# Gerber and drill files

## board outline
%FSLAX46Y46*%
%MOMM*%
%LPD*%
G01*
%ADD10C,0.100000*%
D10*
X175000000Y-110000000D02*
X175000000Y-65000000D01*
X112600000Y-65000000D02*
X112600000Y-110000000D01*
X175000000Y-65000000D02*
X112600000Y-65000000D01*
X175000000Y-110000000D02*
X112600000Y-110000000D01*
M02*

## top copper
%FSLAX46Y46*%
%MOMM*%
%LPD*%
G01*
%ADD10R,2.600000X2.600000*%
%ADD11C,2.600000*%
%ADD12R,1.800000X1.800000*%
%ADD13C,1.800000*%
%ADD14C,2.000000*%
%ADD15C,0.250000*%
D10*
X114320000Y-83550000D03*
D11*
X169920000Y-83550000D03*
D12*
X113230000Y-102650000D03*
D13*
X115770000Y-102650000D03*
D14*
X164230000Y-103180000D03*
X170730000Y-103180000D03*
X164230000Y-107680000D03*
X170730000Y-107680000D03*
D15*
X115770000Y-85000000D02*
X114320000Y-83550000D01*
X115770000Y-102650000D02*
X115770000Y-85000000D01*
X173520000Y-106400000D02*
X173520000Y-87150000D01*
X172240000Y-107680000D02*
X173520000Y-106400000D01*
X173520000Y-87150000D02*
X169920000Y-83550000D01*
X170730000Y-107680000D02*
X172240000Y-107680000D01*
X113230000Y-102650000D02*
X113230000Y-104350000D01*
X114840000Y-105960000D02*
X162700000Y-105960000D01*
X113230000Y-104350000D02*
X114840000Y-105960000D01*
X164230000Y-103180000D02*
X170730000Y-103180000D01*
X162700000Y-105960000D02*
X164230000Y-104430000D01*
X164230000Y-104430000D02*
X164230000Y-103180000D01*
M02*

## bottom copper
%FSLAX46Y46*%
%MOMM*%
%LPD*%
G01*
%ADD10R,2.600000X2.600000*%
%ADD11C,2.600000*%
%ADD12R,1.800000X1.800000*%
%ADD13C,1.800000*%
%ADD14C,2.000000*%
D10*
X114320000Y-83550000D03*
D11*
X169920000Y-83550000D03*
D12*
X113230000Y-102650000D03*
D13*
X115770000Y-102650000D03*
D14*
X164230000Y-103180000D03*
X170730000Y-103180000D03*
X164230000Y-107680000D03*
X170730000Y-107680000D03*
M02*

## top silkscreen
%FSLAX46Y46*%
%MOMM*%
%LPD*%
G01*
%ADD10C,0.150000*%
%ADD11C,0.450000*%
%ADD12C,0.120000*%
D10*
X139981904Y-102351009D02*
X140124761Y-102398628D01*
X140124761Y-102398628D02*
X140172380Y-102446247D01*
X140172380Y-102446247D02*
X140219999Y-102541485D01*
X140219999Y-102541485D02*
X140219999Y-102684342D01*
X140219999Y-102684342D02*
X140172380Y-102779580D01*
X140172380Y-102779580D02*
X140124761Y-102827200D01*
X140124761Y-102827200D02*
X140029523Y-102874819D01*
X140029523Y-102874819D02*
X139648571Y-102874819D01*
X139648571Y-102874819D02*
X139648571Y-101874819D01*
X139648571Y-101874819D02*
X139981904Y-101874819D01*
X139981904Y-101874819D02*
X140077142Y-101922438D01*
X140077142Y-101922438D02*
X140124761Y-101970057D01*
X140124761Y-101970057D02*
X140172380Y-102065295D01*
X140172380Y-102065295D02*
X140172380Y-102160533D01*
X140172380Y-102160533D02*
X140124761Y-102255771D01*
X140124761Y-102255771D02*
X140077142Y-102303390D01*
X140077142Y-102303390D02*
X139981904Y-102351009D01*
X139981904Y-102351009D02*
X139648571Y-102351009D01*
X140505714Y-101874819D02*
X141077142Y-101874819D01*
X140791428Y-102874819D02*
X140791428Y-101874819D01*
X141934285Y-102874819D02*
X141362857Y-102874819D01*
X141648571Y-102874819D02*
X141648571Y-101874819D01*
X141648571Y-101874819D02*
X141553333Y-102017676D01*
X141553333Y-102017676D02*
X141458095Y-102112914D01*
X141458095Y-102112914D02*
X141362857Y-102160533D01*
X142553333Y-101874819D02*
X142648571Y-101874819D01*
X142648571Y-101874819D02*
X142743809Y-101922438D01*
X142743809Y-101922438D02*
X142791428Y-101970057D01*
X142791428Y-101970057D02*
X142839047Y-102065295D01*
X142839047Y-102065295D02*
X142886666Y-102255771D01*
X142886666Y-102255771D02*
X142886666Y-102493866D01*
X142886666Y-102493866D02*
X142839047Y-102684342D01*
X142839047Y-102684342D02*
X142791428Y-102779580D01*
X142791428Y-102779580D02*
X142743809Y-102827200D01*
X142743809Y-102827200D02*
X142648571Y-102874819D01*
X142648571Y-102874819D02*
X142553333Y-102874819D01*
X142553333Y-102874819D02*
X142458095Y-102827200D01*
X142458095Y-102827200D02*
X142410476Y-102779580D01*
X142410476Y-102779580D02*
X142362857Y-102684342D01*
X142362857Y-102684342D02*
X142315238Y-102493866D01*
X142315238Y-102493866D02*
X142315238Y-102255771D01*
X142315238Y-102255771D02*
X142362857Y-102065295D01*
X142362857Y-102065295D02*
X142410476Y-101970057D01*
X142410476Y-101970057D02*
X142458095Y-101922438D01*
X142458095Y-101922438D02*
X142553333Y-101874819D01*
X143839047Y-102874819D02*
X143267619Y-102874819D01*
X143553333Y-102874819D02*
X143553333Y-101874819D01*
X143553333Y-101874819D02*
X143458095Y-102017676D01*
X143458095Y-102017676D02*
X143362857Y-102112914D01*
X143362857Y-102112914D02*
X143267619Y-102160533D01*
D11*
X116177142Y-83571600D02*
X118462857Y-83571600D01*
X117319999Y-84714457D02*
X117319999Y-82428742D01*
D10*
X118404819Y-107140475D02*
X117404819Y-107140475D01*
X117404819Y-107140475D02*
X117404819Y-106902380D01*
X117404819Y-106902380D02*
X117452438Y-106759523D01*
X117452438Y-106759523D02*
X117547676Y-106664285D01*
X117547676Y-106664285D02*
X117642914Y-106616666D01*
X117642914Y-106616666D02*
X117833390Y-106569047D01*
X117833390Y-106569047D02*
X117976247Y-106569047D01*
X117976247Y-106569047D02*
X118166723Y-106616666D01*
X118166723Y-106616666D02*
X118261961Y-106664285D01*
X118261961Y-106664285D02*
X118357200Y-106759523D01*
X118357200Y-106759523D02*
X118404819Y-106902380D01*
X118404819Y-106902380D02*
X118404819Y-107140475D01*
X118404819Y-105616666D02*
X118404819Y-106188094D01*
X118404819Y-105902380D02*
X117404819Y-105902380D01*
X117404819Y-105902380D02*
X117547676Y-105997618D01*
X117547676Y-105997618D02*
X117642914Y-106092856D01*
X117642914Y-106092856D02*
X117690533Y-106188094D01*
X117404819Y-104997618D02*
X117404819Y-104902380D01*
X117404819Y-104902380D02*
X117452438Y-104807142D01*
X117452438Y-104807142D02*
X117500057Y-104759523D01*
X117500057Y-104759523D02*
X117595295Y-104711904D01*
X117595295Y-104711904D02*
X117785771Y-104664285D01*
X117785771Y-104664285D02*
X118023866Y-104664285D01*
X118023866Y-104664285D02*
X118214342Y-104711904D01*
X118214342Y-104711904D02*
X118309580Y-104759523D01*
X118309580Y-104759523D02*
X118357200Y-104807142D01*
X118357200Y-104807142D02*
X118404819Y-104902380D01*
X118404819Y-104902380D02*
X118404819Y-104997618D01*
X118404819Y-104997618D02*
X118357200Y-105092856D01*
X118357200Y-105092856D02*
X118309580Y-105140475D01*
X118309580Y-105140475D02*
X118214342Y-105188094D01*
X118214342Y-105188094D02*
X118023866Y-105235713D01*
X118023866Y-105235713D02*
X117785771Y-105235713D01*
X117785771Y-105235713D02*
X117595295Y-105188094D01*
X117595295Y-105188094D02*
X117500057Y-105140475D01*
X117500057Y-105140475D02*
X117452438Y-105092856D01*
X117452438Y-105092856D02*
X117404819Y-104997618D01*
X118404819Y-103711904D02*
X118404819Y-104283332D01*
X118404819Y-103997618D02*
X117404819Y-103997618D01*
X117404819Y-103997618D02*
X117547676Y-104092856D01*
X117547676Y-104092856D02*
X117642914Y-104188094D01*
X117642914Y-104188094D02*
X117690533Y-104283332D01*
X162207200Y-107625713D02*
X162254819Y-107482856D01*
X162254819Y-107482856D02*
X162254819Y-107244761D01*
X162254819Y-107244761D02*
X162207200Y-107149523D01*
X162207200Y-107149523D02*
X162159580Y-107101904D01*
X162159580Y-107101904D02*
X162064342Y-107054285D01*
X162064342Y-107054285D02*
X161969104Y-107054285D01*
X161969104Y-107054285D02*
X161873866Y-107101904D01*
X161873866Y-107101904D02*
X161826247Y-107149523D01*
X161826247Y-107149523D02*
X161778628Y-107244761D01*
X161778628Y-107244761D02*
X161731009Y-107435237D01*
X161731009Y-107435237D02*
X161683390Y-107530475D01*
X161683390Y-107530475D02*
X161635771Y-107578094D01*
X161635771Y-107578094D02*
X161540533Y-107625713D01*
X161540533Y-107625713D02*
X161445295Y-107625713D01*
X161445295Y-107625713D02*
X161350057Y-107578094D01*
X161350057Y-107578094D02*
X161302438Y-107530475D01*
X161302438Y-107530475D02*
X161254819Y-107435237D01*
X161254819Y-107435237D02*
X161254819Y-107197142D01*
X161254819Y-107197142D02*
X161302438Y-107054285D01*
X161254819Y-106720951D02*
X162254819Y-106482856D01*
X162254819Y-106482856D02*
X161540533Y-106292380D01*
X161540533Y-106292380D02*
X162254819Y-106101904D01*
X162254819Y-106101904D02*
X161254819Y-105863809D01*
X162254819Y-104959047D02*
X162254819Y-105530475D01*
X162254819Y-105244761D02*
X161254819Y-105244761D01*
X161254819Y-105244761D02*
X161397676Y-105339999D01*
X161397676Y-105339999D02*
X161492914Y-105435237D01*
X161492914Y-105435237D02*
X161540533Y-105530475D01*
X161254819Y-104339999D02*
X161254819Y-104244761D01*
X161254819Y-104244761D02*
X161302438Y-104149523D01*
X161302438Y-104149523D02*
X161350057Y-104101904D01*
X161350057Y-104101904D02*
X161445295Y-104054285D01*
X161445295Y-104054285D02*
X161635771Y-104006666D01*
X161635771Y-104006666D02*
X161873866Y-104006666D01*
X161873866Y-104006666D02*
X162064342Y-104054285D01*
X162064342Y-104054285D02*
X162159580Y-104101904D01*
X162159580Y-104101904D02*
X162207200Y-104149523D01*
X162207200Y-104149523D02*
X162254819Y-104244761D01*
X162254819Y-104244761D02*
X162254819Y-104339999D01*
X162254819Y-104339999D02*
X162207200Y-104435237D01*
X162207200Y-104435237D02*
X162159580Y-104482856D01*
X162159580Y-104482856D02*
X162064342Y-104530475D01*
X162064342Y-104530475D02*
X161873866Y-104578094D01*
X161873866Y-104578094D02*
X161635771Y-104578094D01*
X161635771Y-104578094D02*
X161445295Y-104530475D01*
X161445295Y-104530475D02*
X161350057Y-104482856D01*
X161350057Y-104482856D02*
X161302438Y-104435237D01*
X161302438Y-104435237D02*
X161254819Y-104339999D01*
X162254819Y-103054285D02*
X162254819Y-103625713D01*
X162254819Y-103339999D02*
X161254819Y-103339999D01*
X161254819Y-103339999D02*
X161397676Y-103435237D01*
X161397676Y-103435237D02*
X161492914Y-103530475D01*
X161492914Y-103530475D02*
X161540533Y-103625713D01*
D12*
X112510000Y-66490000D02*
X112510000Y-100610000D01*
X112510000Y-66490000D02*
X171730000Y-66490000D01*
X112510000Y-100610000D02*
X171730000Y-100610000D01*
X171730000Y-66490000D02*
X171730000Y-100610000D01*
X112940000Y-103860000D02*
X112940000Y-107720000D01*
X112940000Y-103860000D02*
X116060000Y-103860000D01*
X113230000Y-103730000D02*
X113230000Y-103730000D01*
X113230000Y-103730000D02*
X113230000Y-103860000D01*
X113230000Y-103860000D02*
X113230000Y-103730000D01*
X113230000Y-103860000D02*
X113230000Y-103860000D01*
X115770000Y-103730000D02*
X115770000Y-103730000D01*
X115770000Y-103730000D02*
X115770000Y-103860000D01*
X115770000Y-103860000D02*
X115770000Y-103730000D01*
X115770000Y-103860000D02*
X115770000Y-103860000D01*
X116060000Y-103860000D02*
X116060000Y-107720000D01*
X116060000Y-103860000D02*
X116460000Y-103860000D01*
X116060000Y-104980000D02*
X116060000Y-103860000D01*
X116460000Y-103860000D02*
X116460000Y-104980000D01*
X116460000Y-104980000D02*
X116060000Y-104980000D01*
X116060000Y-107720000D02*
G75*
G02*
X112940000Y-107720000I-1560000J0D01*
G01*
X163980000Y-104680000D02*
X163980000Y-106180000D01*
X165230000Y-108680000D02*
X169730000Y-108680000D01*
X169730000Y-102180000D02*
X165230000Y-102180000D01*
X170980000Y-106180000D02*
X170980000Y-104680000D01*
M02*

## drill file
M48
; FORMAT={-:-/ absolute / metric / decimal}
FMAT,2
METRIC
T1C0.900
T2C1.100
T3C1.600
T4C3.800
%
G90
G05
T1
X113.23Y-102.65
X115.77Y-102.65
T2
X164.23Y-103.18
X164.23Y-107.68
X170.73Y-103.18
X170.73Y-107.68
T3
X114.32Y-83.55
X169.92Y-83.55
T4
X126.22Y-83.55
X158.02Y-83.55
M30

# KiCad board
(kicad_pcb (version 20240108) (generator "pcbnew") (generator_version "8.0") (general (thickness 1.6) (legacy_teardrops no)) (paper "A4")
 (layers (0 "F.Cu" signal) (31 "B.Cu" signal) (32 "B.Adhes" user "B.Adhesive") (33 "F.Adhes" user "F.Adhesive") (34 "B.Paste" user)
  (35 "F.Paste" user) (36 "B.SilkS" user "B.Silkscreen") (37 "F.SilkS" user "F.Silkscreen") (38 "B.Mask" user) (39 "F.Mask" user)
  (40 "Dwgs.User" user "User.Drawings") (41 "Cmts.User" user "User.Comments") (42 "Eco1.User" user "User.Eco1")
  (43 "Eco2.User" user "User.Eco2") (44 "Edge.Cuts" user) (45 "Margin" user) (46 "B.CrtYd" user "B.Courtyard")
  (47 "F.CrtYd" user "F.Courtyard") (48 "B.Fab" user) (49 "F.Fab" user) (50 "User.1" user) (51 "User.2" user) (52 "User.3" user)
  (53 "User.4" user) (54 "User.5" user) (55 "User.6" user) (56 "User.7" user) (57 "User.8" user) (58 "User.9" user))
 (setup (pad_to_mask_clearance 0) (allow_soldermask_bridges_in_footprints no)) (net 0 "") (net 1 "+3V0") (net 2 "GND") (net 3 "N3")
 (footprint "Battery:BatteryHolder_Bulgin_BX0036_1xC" (layer "F.Cu") (at 114.32 83.55)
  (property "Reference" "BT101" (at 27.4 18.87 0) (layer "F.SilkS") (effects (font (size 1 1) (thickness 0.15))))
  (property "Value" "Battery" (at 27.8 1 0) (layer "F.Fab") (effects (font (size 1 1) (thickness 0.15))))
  (fp_line (start -1.81 -17.06) (end -1.81 17.06) (stroke (width 0.12) (type solid)) (layer "F.SilkS"))
  (fp_line (start -1.81 -17.06) (end 57.41 -17.06) (stroke (width 0.12) (type solid)) (layer "F.SilkS"))
  (fp_line (start -1.81 17.06) (end 57.41 17.06) (stroke (width 0.12) (type solid)) (layer "F.SilkS"))
  (fp_line (start 57.41 -17.06) (end 57.41 17.06) (stroke (width 0.12) (type solid)) (layer "F.SilkS"))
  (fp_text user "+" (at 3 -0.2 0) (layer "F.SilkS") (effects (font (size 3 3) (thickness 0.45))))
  (pad "" np_thru_hole circle (at 11.9 0) (size 3.8 3.8) (drill 3.8) (layers "*.Cu" "*.Mask"))
  (pad "" np_thru_hole circle (at 43.7 0) (size 3.8 3.8) (drill 3.8) (layers "*.Cu" "*.Mask"))
  (pad "1" thru_hole rect (at 0 0) (size 2.6 2.6) (drill 1.6) (layers "*.Cu" "*.Mask") (remove_unused_layers no) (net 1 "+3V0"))
  (pad "2" thru_hole circle (at 55.6 0) (size 2.6 2.6) (drill 1.6) (layers "*.Cu" "*.Mask") (remove_unused_layers no) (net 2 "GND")))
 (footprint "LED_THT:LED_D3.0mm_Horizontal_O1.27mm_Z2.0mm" (layer "F.Cu") (at 113.23 102.65)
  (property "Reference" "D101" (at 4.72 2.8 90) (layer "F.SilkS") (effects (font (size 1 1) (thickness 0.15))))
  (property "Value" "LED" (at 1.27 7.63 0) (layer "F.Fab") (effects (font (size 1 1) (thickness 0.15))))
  (fp_line (start -0.29 1.21) (end -0.29 5.07) (stroke (width 0.12) (type solid)) (layer "F.SilkS"))
  (fp_line (start -0.29 1.21) (end 2.83 1.21) (stroke (width 0.12) (type solid)) (layer "F.SilkS"))
  (fp_line (start 0 1.08) (end 0 1.08) (stroke (width 0.12) (type solid)) (layer "F.SilkS"))
  (fp_line (start 0 1.08) (end 0 1.21) (stroke (width 0.12) (type solid)) (layer "F.SilkS"))
  (fp_line (start 0 1.21) (end 0 1.08) (stroke (width 0.12) (type solid)) (layer "F.SilkS"))
  (fp_line (start 0 1.21) (end 0 1.21) (stroke (width 0.12) (type solid)) (layer "F.SilkS"))
  (fp_line (start 2.54 1.08) (end 2.54 1.08) (stroke (width 0.12) (type solid)) (layer "F.SilkS"))
  (fp_line (start 2.54 1.08) (end 2.54 1.21) (stroke (width 0.12) (type solid)) (layer "F.SilkS"))
  (fp_line (start 2.54 1.21) (end 2.54 1.08) (stroke (width 0.12) (type solid)) (layer "F.SilkS"))
  (fp_line (start 2.54 1.21) (end 2.54 1.21) (stroke (width 0.12) (type solid)) (layer "F.SilkS"))
  (fp_line (start 2.83 1.21) (end 2.83 5.07) (stroke (width 0.12) (type solid)) (layer "F.SilkS"))
  (fp_line (start 2.83 1.21) (end 3.23 1.21) (stroke (width 0.12) (type solid)) (layer "F.SilkS"))
  (fp_line (start 2.83 2.33) (end 2.83 1.21) (stroke (width 0.12) (type solid)) (layer "F.SilkS"))
  (fp_line (start 3.23 1.21) (end 3.23 2.33) (stroke (width 0.12) (type solid)) (layer "F.SilkS"))
  (fp_line (start 3.23 2.33) (end 2.83 2.33) (stroke (width 0.12) (type solid)) (layer "F.SilkS"))
  (fp_arc (start 2.83 5.07) (mid 1.27 6.63) (end -0.29 5.07) (stroke (width 0.12) (type solid)) (layer "F.SilkS"))
  (pad "1" thru_hole rect (at 0 0) (size 1.8 1.8) (drill 0.9) (layers "*.Cu" "*.Mask") (remove_unused_layers no) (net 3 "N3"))
  (pad "2" thru_hole circle (at 2.54 0) (size 1.8 1.8) (drill 0.9) (layers "*.Cu" "*.Mask") (remove_unused_layers no) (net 1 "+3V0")))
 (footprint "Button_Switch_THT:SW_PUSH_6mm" (layer "F.Cu") (at 164.23 103.18)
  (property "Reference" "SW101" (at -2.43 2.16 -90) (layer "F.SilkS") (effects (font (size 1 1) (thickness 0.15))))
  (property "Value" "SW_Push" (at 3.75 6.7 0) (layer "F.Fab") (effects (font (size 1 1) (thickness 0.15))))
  (fp_line (start -0.25 1.5) (end -0.25 3) (stroke (width 0.12) (type solid)) (layer "F.SilkS"))
  (fp_line (start 1 5.5) (end 5.5 5.5) (stroke (width 0.12) (type solid)) (layer "F.SilkS"))
  (fp_line (start 5.5 -1) (end 1 -1) (stroke (width 0.12) (type solid)) (layer "F.SilkS"))
  (fp_line (start 6.75 3) (end 6.75 1.5) (stroke (width 0.12) (type solid)) (layer "F.SilkS"))
  (pad "1" thru_hole circle (at 0 0 90) (size 2 2) (drill 1.1) (layers "*.Cu" "*.Mask") (remove_unused_layers no) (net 3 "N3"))
  (pad "1" thru_hole circle (at 6.5 0 90) (size 2 2) (drill 1.1) (layers "*.Cu" "*.Mask") (remove_unused_layers no) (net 3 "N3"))
  (pad "2" thru_hole circle (at 0 4.5 90) (size 2 2) (drill 1.1) (layers "*.Cu" "*.Mask") (remove_unused_layers no) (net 2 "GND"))
  (pad "2" thru_hole circle (at 6.5 4.5 90) (size 2 2) (drill 1.1) (layers "*.Cu" "*.Mask") (remove_unused_layers no) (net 2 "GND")))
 (gr_line (start 175 110) (end 175 65) (stroke (width 0.1) (type default)) (layer "Edge.Cuts"))
 (gr_line (start 112.6 65) (end 112.6 110) (stroke (width 0.1) (type default)) (layer "Edge.Cuts"))
 (gr_line (start 175 65) (end 112.6 65) (stroke (width 0.1) (type default)) (layer "Edge.Cuts"))
 (gr_line (start 175 110) (end 112.6 110) (stroke (width 0.1) (type default)) (layer "Edge.Cuts"))
 (segment (start 115.77 85) (end 114.32 83.55) (width 0.25) (layer "F.Cu") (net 1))
 (segment (start 115.77 102.65) (end 115.77 85) (width 0.25) (layer "F.Cu") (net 1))
 (segment (start 173.52 106.4) (end 173.52 87.15) (width 0.25) (layer "F.Cu") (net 2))
 (segment (start 172.24 107.68) (end 173.52 106.4) (width 0.25) (layer "F.Cu") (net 2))
 (segment (start 173.52 87.15) (end 169.92 83.55) (width 0.25) (layer "F.Cu") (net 2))
 (segment (start 170.73 107.68) (end 172.24 107.68) (width 0.25) (layer "F.Cu") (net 2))
 (segment (start 113.23 102.65) (end 113.23 104.35) (width 0.25) (layer "F.Cu") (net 3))
 (segment (start 114.84 105.96) (end 162.7 105.96) (width 0.25) (layer "F.Cu") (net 3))
 (segment (start 113.23 104.35) (end 114.84 105.96) (width 0.25) (layer "F.Cu") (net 3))
 (segment (start 164.23 103.18) (end 170.73 103.18) (width 0.25) (layer "F.Cu") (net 3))
 (segment (start 162.7 105.96) (end 164.23 104.43) (width 0.25) (layer "F.Cu") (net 3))
 (segment (start 164.23 104.43) (end 164.23 103.18) (width 0.25) (layer "F.Cu") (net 3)))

